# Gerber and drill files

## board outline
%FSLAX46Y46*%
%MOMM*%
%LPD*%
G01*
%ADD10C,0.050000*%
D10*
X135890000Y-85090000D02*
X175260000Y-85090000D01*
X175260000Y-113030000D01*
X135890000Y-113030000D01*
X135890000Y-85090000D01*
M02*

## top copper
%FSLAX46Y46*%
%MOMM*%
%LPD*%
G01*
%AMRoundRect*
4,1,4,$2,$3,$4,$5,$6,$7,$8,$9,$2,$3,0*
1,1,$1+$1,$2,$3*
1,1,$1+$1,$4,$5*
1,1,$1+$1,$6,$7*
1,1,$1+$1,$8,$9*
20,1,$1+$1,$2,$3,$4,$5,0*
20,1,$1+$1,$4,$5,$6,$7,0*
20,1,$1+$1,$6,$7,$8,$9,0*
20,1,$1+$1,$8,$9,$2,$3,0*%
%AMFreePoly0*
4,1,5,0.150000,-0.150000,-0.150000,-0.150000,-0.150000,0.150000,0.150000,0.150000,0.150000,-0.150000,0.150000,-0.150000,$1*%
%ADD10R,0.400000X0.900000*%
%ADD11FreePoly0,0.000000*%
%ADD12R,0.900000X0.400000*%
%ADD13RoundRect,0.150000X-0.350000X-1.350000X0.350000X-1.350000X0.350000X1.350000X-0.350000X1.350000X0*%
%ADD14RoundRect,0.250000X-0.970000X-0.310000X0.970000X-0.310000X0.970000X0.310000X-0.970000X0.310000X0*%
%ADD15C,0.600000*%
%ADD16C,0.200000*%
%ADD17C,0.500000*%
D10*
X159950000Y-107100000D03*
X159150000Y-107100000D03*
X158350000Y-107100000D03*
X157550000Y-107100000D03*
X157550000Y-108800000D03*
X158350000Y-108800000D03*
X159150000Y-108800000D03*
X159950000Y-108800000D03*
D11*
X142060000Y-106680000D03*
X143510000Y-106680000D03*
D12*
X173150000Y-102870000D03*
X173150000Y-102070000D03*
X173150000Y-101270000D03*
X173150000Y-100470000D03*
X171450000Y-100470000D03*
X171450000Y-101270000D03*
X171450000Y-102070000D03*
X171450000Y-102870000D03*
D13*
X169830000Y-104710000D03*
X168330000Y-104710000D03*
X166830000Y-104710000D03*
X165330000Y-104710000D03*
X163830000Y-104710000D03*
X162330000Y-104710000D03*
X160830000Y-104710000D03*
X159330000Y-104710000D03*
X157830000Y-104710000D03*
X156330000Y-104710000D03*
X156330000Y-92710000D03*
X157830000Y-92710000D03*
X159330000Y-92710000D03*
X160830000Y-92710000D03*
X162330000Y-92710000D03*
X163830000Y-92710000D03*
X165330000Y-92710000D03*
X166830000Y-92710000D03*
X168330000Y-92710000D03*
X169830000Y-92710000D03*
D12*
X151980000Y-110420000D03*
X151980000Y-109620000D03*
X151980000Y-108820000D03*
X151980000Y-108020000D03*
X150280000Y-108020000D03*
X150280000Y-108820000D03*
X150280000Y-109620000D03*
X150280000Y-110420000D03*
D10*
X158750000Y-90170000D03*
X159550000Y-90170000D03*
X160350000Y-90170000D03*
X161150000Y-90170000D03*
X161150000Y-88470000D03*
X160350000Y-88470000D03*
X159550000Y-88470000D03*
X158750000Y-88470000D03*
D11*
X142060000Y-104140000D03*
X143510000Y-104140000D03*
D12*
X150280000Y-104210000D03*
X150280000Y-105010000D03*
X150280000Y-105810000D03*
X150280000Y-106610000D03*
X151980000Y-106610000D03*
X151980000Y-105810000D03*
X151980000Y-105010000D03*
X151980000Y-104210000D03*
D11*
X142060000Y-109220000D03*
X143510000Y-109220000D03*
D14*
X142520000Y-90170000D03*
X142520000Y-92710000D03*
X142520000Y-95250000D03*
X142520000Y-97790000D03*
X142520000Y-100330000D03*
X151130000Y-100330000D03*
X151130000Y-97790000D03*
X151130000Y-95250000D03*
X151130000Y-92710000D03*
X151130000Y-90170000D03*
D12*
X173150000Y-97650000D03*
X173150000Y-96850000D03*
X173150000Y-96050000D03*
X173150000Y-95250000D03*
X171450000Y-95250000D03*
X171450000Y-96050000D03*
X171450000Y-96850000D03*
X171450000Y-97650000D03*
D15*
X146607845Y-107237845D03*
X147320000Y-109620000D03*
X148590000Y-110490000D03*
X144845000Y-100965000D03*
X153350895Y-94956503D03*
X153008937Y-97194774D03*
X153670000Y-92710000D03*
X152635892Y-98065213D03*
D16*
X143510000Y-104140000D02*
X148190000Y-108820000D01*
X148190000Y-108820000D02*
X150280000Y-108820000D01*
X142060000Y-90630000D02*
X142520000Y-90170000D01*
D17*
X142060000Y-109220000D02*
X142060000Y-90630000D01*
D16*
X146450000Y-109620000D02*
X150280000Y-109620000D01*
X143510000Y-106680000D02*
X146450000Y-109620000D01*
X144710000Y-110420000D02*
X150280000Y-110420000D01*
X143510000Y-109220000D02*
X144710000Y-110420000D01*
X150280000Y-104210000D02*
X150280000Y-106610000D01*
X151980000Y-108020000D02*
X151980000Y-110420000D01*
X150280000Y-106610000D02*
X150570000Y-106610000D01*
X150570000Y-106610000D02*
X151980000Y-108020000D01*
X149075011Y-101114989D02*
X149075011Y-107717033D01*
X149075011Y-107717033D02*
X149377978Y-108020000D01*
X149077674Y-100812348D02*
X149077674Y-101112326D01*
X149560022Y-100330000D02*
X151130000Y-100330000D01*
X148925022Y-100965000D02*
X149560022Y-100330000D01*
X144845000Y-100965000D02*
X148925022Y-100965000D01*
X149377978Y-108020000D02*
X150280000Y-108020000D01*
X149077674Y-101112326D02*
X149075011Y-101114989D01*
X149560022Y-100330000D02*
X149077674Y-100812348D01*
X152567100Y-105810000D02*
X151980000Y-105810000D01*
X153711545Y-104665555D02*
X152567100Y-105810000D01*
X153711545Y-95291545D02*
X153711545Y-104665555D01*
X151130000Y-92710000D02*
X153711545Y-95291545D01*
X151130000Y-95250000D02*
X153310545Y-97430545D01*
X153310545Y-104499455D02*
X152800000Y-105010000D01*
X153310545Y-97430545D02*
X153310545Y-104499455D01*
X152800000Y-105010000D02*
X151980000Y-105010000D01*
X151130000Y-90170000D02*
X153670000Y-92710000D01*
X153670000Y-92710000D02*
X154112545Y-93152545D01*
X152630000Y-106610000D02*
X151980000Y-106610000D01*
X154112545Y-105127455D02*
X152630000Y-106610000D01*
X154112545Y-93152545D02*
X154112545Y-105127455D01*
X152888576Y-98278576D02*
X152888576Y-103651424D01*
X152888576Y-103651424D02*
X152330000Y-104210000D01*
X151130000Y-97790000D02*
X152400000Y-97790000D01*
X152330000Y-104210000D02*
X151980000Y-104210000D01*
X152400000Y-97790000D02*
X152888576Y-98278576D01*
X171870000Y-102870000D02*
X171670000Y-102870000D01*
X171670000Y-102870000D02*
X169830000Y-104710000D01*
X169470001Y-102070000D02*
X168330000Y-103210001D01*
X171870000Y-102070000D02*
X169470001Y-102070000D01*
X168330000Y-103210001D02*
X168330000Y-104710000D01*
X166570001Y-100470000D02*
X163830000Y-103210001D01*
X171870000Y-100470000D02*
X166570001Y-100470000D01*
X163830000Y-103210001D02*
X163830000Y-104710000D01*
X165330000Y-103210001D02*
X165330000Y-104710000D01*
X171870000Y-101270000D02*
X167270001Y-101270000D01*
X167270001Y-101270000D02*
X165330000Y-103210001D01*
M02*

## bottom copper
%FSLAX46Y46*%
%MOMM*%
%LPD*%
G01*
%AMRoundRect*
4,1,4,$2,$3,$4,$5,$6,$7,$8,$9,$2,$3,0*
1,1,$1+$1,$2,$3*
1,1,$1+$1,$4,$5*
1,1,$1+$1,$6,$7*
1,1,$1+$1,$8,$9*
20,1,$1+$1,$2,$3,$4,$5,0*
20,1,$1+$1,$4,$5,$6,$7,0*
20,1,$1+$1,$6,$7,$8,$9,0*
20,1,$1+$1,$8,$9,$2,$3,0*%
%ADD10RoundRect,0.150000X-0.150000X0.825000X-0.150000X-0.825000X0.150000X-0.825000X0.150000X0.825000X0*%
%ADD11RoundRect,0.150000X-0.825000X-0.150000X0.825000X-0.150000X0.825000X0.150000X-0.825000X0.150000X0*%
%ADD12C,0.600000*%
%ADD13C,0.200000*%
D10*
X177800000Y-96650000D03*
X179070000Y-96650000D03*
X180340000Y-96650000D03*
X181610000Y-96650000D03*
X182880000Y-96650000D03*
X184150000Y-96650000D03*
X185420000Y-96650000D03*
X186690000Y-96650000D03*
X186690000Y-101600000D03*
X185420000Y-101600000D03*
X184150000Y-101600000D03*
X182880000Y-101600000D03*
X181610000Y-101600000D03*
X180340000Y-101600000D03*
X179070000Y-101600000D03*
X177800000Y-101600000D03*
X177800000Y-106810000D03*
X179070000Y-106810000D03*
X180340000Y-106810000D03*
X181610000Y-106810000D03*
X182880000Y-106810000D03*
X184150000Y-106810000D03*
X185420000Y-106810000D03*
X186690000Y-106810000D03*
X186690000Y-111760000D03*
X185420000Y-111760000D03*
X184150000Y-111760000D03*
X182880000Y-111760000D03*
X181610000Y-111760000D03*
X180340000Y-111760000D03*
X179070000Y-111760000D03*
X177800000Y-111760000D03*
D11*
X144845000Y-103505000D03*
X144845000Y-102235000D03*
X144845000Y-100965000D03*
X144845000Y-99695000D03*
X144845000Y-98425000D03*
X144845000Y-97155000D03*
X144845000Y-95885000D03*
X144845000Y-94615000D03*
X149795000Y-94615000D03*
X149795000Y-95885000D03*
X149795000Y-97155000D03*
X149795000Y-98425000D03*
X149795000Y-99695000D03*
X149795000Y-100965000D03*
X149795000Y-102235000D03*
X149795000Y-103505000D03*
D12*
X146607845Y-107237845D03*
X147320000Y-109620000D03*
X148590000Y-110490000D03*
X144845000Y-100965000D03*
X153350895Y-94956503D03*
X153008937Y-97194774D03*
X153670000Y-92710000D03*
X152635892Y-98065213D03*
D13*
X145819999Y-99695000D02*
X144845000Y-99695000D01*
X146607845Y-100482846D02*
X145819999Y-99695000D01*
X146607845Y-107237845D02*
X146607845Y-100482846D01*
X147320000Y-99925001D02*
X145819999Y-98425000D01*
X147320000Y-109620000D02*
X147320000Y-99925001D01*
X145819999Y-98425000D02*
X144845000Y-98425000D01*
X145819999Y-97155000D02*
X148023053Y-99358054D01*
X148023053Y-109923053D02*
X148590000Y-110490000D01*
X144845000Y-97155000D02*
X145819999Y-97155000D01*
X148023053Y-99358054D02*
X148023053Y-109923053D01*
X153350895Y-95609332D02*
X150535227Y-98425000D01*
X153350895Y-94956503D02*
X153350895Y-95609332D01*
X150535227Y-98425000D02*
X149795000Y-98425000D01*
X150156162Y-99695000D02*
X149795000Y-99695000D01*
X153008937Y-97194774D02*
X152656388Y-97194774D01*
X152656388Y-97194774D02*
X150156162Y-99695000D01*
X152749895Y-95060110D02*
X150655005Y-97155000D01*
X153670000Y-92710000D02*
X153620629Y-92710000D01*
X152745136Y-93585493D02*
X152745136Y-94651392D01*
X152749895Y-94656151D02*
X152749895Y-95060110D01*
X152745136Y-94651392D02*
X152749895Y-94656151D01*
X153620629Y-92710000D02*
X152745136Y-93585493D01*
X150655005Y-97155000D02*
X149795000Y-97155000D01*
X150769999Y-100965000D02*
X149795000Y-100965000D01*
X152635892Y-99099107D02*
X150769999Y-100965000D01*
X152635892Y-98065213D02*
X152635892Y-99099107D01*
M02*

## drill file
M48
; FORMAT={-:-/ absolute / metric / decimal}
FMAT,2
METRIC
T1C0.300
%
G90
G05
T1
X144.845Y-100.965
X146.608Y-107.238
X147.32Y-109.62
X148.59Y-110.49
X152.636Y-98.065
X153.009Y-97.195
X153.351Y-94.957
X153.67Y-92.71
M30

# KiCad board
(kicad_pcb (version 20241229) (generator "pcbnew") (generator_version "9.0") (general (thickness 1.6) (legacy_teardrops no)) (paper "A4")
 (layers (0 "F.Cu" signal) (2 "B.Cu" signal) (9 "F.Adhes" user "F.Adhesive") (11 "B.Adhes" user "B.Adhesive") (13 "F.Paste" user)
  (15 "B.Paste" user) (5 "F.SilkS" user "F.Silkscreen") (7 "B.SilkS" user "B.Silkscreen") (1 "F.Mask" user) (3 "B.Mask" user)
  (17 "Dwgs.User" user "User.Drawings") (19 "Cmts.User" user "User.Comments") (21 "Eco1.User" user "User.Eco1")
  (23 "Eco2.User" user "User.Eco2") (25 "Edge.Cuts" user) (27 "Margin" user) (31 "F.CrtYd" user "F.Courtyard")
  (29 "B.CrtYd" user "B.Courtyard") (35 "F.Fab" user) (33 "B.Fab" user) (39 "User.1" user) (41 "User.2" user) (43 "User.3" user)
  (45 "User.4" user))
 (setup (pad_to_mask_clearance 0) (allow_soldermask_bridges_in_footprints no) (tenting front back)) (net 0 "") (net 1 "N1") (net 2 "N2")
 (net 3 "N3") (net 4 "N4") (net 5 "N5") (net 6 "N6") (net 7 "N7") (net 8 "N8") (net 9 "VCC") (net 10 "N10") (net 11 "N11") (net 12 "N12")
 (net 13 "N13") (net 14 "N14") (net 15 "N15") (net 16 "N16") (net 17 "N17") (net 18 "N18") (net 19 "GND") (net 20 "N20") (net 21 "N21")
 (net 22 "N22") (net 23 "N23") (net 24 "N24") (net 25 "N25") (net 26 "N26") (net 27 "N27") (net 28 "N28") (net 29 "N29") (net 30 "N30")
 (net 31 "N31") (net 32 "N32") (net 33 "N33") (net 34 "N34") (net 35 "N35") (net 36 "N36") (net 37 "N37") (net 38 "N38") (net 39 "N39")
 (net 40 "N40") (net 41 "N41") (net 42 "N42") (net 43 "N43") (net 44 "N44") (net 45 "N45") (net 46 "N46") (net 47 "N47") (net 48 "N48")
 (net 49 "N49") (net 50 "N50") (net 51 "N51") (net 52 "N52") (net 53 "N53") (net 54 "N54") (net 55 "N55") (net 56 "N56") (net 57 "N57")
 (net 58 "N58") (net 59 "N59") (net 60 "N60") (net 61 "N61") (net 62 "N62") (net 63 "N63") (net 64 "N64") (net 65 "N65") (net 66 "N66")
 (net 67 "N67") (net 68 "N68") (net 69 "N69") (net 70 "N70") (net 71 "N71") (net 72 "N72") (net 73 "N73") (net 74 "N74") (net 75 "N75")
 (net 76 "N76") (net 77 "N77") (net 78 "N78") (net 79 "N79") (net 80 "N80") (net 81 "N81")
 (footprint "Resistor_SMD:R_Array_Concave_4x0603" (layer "F.Cu") (at 158.75 107.95 -90)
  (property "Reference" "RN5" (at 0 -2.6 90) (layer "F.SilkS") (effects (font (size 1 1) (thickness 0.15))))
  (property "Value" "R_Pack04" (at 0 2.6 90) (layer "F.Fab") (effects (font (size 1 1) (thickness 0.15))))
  (pad "1" smd rect (at -0.85 -1.2 270) (size 0.9 0.4) (layers "F.Cu" "F.Mask" "F.Paste") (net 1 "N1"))
  (pad "2" smd rect (at -0.85 -0.4 270) (size 0.9 0.4) (layers "F.Cu" "F.Mask" "F.Paste") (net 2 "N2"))
  (pad "3" smd rect (at -0.85 0.4 270) (size 0.9 0.4) (layers "F.Cu" "F.Mask" "F.Paste") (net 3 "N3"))
  (pad "4" smd rect (at -0.85 1.2 270) (size 0.9 0.4) (layers "F.Cu" "F.Mask" "F.Paste") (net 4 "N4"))
  (pad "5" smd rect (at 0.85 1.2 270) (size 0.9 0.4) (layers "F.Cu" "F.Mask" "F.Paste") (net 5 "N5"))
  (pad "6" smd rect (at 0.85 0.4 270) (size 0.9 0.4) (layers "F.Cu" "F.Mask" "F.Paste") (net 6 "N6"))
  (pad "7" smd rect (at 0.85 -0.4 270) (size 0.9 0.4) (layers "F.Cu" "F.Mask" "F.Paste") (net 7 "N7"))
  (pad "8" smd rect (at 0.85 -1.2 270) (size 0.9 0.4) (layers "F.Cu" "F.Mask" "F.Paste") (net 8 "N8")))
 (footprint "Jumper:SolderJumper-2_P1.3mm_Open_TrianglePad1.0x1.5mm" (layer "F.Cu") (at 142.785 106.68)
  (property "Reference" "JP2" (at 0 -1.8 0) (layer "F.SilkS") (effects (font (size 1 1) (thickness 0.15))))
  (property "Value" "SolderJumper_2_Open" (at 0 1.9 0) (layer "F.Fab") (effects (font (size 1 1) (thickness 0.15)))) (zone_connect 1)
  (pad "1" smd custom (at -0.725 0) (size 0.3 0.3) (layers "F.Cu" "F.Mask") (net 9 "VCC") (zone_connect 2) (thermal_bridge_angle 45)
   (options (clearance outline) (anchor rect)) (primitives))
  (pad "2" smd custom (at 0.725 0) (size 0.3 0.3) (layers "F.Cu" "F.Mask") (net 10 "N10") (zone_connect 2) (thermal_bridge_angle 45)
   (options (clearance outline) (anchor rect)) (primitives)))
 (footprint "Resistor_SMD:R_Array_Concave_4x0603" (layer "F.Cu") (at 172.3 101.67 180)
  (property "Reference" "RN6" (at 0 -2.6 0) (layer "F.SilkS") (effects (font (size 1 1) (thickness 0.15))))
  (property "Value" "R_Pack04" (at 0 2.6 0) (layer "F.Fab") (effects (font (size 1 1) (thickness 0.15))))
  (pad "1" smd rect (at -0.85 -1.2 180) (size 0.9 0.4) (layers "F.Cu" "F.Mask" "F.Paste") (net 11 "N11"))
  (pad "2" smd rect (at -0.85 -0.4 180) (size 0.9 0.4) (layers "F.Cu" "F.Mask" "F.Paste") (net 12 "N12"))
  (pad "3" smd rect (at -0.85 0.4 180) (size 0.9 0.4) (layers "F.Cu" "F.Mask" "F.Paste") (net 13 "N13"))
  (pad "4" smd rect (at -0.85 1.2 180) (size 0.9 0.4) (layers "F.Cu" "F.Mask" "F.Paste") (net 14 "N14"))
  (pad "5" smd rect (at 0.85 1.2 180) (size 0.9 0.4) (layers "F.Cu" "F.Mask" "F.Paste") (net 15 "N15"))
  (pad "6" smd rect (at 0.85 0.4 180) (size 0.9 0.4) (layers "F.Cu" "F.Mask" "F.Paste") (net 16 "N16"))
  (pad "7" smd rect (at 0.85 -0.4 180) (size 0.9 0.4) (layers "F.Cu" "F.Mask" "F.Paste") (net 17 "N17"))
  (pad "8" smd rect (at 0.85 -1.2 180) (size 0.9 0.4) (layers "F.Cu" "F.Mask" "F.Paste") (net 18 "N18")))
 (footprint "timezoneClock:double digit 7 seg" (layer "F.Cu") (at 163.08 98.71)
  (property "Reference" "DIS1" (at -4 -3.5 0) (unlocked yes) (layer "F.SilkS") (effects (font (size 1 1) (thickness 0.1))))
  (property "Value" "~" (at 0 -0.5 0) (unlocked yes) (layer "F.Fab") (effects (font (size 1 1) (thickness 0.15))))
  (pad "1" smd roundrect (at 6.75 6) (size 1 3) (layers "F.Cu" "F.Mask" "F.Paste") (roundrect_rratio 0.15) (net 18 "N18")
   (thermal_bridge_angle 45))
  (pad "2" smd roundrect (at 5.25 6) (size 1 3) (layers "F.Cu" "F.Mask" "F.Paste") (roundrect_rratio 0.15) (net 17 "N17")
   (thermal_bridge_angle 45))
  (pad "3" smd roundrect (at 3.75 6) (size 1 3) (layers "F.Cu" "F.Mask" "F.Paste") (roundrect_rratio 0.15) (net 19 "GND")
   (thermal_bridge_angle 45))
  (pad "4" smd roundrect (at 2.25 6) (size 1 3) (layers "F.Cu" "F.Mask" "F.Paste") (roundrect_rratio 0.15) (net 16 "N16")
   (thermal_bridge_angle 45))
  (pad "5" smd roundrect (at 0.75 6) (size 1 3) (layers "F.Cu" "F.Mask" "F.Paste") (roundrect_rratio 0.15) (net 15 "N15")
   (thermal_bridge_angle 45))
  (pad "6" smd roundrect (at -0.75 6) (size 1 3) (layers "F.Cu" "F.Mask" "F.Paste") (roundrect_rratio 0.15) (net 8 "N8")
   (thermal_bridge_angle 45))
  (pad "7" smd roundrect (at -2.25 6) (size 1 3) (layers "F.Cu" "F.Mask" "F.Paste") (roundrect_rratio 0.15) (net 7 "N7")
   (thermal_bridge_angle 45))
  (pad "8" smd roundrect (at -3.75 6) (size 1 3) (layers "F.Cu" "F.Mask" "F.Paste") (roundrect_rratio 0.15) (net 19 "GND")
   (thermal_bridge_angle 45))
  (pad "9" smd roundrect (at -5.25 6) (size 1 3) (layers "F.Cu" "F.Mask" "F.Paste") (roundrect_rratio 0.15) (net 6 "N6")
   (thermal_bridge_angle 45))
  (pad "10" smd roundrect (at -6.75 6) (size 1 3) (layers "F.Cu" "F.Mask" "F.Paste") (roundrect_rratio 0.15) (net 5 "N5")
   (thermal_bridge_angle 45))
  (pad "11" smd roundrect (at -6.75 -6) (size 1 3) (layers "F.Cu" "F.Mask" "F.Paste") (roundrect_rratio 0.15) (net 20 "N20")
   (thermal_bridge_angle 45))
  (pad "12" smd roundrect (at -5.25 -6) (size 1 3) (layers "F.Cu" "F.Mask" "F.Paste") (roundrect_rratio 0.15) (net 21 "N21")
   (thermal_bridge_angle 45))
  (pad "13" smd roundrect (at -3.75 -6) (size 1 3) (layers "F.Cu" "F.Mask" "F.Paste") (roundrect_rratio 0.15) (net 19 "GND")
   (thermal_bridge_angle 45))
  (pad "14" smd roundrect (at -2.25 -6) (size 1 3) (layers "F.Cu" "F.Mask" "F.Paste") (roundrect_rratio 0.15) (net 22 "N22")
   (thermal_bridge_angle 45))
  (pad "15" smd roundrect (at -0.75 -6) (size 1 3) (layers "F.Cu" "F.Mask" "F.Paste") (roundrect_rratio 0.15) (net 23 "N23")
   (thermal_bridge_angle 45))
  (pad "16" smd roundrect (at 0.75 -6) (size 1 3) (layers "F.Cu" "F.Mask" "F.Paste") (roundrect_rratio 0.15) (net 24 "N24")
   (thermal_bridge_angle 45))
  (pad "17" smd roundrect (at 2.25 -6) (size 1 3) (layers "F.Cu" "F.Mask" "F.Paste") (roundrect_rratio 0.15) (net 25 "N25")
   (thermal_bridge_angle 45))
  (pad "18" smd roundrect (at 3.75 -6) (size 1 3) (layers "F.Cu" "F.Mask" "F.Paste") (roundrect_rratio 0.15) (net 19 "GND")
   (thermal_bridge_angle 45))
  (pad "19" smd roundrect (at 5.25 -6) (size 1 3) (layers "F.Cu" "F.Mask" "F.Paste") (roundrect_rratio 0.15) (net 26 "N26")
   (thermal_bridge_angle 45))
  (pad "20" smd roundrect (at 6.75 -6) (size 1 3) (layers "F.Cu" "F.Mask" "F.Paste") (roundrect_rratio 0.15) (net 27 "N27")
   (thermal_bridge_angle 45)))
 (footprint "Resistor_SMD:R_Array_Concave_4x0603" (layer "F.Cu") (at 151.13 109.22 180)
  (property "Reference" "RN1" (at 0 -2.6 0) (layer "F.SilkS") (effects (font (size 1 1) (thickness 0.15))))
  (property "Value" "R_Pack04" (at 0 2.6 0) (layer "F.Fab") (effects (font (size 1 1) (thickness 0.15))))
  (pad "1" smd rect (at -0.85 -1.2 180) (size 0.9 0.4) (layers "F.Cu" "F.Mask" "F.Paste") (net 19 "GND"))
  (pad "2" smd rect (at -0.85 -0.4 180) (size 0.9 0.4) (layers "F.Cu" "F.Mask" "F.Paste") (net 19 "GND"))
  (pad "3" smd rect (at -0.85 0.4 180) (size 0.9 0.4) (layers "F.Cu" "F.Mask" "F.Paste") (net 19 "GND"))
  (pad "4" smd rect (at -0.85 1.2 180) (size 0.9 0.4) (layers "F.Cu" "F.Mask" "F.Paste") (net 19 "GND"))
  (pad "5" smd rect (at 0.85 1.2 180) (size 0.9 0.4) (layers "F.Cu" "F.Mask" "F.Paste") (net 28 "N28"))
  (pad "6" smd rect (at 0.85 0.4 180) (size 0.9 0.4) (layers "F.Cu" "F.Mask" "F.Paste") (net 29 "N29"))
  (pad "7" smd rect (at 0.85 -0.4 180) (size 0.9 0.4) (layers "F.Cu" "F.Mask" "F.Paste") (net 10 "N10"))
  (pad "8" smd rect (at 0.85 -1.2 180) (size 0.9 0.4) (layers "F.Cu" "F.Mask" "F.Paste") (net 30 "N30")))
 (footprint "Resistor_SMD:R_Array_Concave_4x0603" (layer "F.Cu") (at 159.95 89.32 90)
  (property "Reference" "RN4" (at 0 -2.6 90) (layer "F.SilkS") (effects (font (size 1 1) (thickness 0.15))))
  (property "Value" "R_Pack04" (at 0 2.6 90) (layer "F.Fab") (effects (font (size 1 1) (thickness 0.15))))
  (pad "1" smd rect (at -0.85 -1.2 90) (size 0.9 0.4) (layers "F.Cu" "F.Mask" "F.Paste") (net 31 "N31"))
  (pad "2" smd rect (at -0.85 -0.4 90) (size 0.9 0.4) (layers "F.Cu" "F.Mask" "F.Paste") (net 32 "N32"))
  (pad "3" smd rect (at -0.85 0.4 90) (size 0.9 0.4) (layers "F.Cu" "F.Mask" "F.Paste") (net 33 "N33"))
  (pad "4" smd rect (at -0.85 1.2 90) (size 0.9 0.4) (layers "F.Cu" "F.Mask" "F.Paste") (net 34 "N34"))
  (pad "5" smd rect (at 0.85 1.2 90) (size 0.9 0.4) (layers "F.Cu" "F.Mask" "F.Paste") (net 23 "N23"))
  (pad "6" smd rect (at 0.85 0.4 90) (size 0.9 0.4) (layers "F.Cu" "F.Mask" "F.Paste") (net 22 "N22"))
  (pad "7" smd rect (at 0.85 -0.4 90) (size 0.9 0.4) (layers "F.Cu" "F.Mask" "F.Paste") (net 21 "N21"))
  (pad "8" smd rect (at 0.85 -1.2 90) (size 0.9 0.4) (layers "F.Cu" "F.Mask" "F.Paste") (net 20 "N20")))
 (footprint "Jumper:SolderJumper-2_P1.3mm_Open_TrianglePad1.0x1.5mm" (layer "F.Cu") (at 142.785 104.14)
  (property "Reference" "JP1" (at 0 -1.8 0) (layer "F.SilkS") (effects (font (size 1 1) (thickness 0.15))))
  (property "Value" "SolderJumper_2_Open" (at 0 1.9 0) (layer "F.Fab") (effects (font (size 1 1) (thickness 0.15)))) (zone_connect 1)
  (pad "1" smd custom (at -0.725 0) (size 0.3 0.3) (layers "F.Cu" "F.Mask") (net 9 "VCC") (zone_connect 2) (thermal_bridge_angle 45)
   (options (clearance outline) (anchor rect)) (primitives))
  (pad "2" smd custom (at 0.725 0) (size 0.3 0.3) (layers "F.Cu" "F.Mask") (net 29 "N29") (zone_connect 2) (thermal_bridge_angle 45)
   (options (clearance outline) (anchor rect)) (primitives)))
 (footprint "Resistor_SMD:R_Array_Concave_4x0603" (layer "F.Cu") (at 151.13 105.41)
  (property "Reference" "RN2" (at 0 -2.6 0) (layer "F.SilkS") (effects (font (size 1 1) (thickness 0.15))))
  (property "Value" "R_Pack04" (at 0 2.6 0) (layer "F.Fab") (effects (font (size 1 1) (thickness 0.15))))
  (pad "1" smd rect (at -0.85 -1.2) (size 0.9 0.4) (layers "F.Cu" "F.Mask" "F.Paste") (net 19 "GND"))
  (pad "2" smd rect (at -0.85 -0.4) (size 0.9 0.4) (layers "F.Cu" "F.Mask" "F.Paste") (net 19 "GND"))
  (pad "3" smd rect (at -0.85 0.4) (size 0.9 0.4) (layers "F.Cu" "F.Mask" "F.Paste") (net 19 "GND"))
  (pad "4" smd rect (at -0.85 1.2) (size 0.9 0.4) (layers "F.Cu" "F.Mask" "F.Paste") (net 19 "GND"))
  (pad "5" smd rect (at 0.85 1.2) (size 0.9 0.4) (layers "F.Cu" "F.Mask" "F.Paste") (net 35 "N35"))
  (pad "6" smd rect (at 0.85 0.4) (size 0.9 0.4) (layers "F.Cu" "F.Mask" "F.Paste") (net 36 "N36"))
  (pad "7" smd rect (at 0.85 -0.4) (size 0.9 0.4) (layers "F.Cu" "F.Mask" "F.Paste") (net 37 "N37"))
  (pad "8" smd rect (at 0.85 -1.2) (size 0.9 0.4) (layers "F.Cu" "F.Mask" "F.Paste") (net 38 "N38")))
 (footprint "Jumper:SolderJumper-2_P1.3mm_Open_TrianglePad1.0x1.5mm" (layer "F.Cu") (at 142.785 109.22)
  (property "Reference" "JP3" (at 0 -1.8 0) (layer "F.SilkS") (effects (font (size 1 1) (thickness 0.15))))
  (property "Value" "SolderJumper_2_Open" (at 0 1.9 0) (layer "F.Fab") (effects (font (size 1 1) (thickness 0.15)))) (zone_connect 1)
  (pad "1" smd custom (at -0.725 0) (size 0.3 0.3) (layers "F.Cu" "F.Mask") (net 9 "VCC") (zone_connect 2) (thermal_bridge_angle 45)
   (options (clearance outline) (anchor rect)) (primitives))
  (pad "2" smd custom (at 0.725 0) (size 0.3 0.3) (layers "F.Cu" "F.Mask") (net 30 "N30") (zone_connect 2) (thermal_bridge_angle 45)
   (options (clearance outline) (anchor rect)) (primitives)))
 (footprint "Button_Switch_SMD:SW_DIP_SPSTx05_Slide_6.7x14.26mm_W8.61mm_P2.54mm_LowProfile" (layer "F.Cu") (at 146.825 95.25)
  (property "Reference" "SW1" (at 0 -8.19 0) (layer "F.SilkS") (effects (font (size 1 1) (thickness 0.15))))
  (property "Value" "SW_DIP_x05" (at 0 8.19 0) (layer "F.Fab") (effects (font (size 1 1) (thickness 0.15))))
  (pad "1" smd roundrect (at -4.305 -5.08) (size 2.44 1.12) (layers "F.Cu" "F.Mask" "F.Paste") (roundrect_rratio 0.223214) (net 9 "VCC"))
  (pad "2" smd roundrect (at -4.305 -2.54) (size 2.44 1.12) (layers "F.Cu" "F.Mask" "F.Paste") (roundrect_rratio 0.223214) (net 9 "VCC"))
  (pad "3" smd roundrect (at -4.305 0) (size 2.44 1.12) (layers "F.Cu" "F.Mask" "F.Paste") (roundrect_rratio 0.223214) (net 9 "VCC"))
  (pad "4" smd roundrect (at -4.305 2.54) (size 2.44 1.12) (layers "F.Cu" "F.Mask" "F.Paste") (roundrect_rratio 0.223214) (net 9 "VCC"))
  (pad "5" smd roundrect (at -4.305 5.08) (size 2.44 1.12) (layers "F.Cu" "F.Mask" "F.Paste") (roundrect_rratio 0.223214) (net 9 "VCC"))
  (pad "6" smd roundrect (at 4.305 5.08) (size 2.44 1.12) (layers "F.Cu" "F.Mask" "F.Paste") (roundrect_rratio 0.223214) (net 28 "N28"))
  (pad "7" smd roundrect (at 4.305 2.54) (size 2.44 1.12) (layers "F.Cu" "F.Mask" "F.Paste") (roundrect_rratio 0.223214) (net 38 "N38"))
  (pad "8" smd roundrect (at 4.305 0) (size 2.44 1.12) (layers "F.Cu" "F.Mask" "F.Paste") (roundrect_rratio 0.223214) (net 37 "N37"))
  (pad "9" smd roundrect (at 4.305 -2.54) (size 2.44 1.12) (layers "F.Cu" "F.Mask" "F.Paste") (roundrect_rratio 0.223214) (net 36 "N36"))
  (pad "10" smd roundrect (at 4.305 -5.08) (size 2.44 1.12) (layers "F.Cu" "F.Mask" "F.Paste") (roundrect_rratio 0.223214) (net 35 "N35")))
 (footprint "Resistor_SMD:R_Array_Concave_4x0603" (layer "F.Cu") (at 172.3 96.45 180)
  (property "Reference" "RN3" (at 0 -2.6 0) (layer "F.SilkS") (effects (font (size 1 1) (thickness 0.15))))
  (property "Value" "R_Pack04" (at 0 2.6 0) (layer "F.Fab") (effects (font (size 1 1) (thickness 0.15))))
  (pad "1" smd rect (at -0.85 -1.2 180) (size 0.9 0.4) (layers "F.Cu" "F.Mask" "F.Paste") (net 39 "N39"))
  (pad "2" smd rect (at -0.85 -0.4 180) (size 0.9 0.4) (layers "F.Cu" "F.Mask" "F.Paste") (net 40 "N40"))
  (pad "3" smd rect (at -0.85 0.4 180) (size 0.9 0.4) (layers "F.Cu" "F.Mask" "F.Paste") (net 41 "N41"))
  (pad "4" smd rect (at -0.85 1.2 180) (size 0.9 0.4) (layers "F.Cu" "F.Mask" "F.Paste") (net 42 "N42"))
  (pad "5" smd rect (at 0.85 1.2 180) (size 0.9 0.4) (layers "F.Cu" "F.Mask" "F.Paste") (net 27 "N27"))
  (pad "6" smd rect (at 0.85 0.4 180) (size 0.9 0.4) (layers "F.Cu" "F.Mask" "F.Paste") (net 26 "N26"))
  (pad "7" smd rect (at 0.85 -0.4 180) (size 0.9 0.4) (layers "F.Cu" "F.Mask" "F.Paste") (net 25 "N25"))
  (pad "8" smd rect (at 0.85 -1.2 180) (size 0.9 0.4) (layers "F.Cu" "F.Mask" "F.Paste") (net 24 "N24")))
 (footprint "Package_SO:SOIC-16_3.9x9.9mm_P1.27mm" (layer "B.Cu") (at 182.245 99.125 -90)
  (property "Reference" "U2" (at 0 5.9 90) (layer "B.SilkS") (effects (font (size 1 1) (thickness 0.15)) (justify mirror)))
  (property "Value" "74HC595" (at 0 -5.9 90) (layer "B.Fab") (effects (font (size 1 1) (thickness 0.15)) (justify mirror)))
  (pad "1" smd roundrect (at -2.475 4.445 270) (size 1.95 0.6) (layers "B.Cu" "B.Mask" "B.Paste") (roundrect_rratio 0.25) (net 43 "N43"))
  (pad "2" smd roundrect (at -2.475 3.175 270) (size 1.95 0.6) (layers "B.Cu" "B.Mask" "B.Paste") (roundrect_rratio 0.25) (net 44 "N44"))
  (pad "3" smd roundrect (at -2.475 1.905 270) (size 1.95 0.6) (layers "B.Cu" "B.Mask" "B.Paste") (roundrect_rratio 0.25) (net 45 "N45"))
  (pad "4" smd roundrect (at -2.475 0.635 270) (size 1.95 0.6) (layers "B.Cu" "B.Mask" "B.Paste") (roundrect_rratio 0.25) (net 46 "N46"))
  (pad "5" smd roundrect (at -2.475 -0.635 270) (size 1.95 0.6) (layers "B.Cu" "B.Mask" "B.Paste") (roundrect_rratio 0.25) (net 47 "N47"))
  (pad "6" smd roundrect (at -2.475 -1.905 270) (size 1.95 0.6) (layers "B.Cu" "B.Mask" "B.Paste") (roundrect_rratio 0.25) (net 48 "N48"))
  (pad "7" smd roundrect (at -2.475 -3.175 270) (size 1.95 0.6) (layers "B.Cu" "B.Mask" "B.Paste") (roundrect_rratio 0.25) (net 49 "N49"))
  (pad "8" smd roundrect (at -2.475 -4.445 270) (size 1.95 0.6) (layers "B.Cu" "B.Mask" "B.Paste") (roundrect_rratio 0.25) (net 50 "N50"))
  (pad "9" smd roundrect (at 2.475 -4.445 270) (size 1.95 0.6) (layers "B.Cu" "B.Mask" "B.Paste") (roundrect_rratio 0.25) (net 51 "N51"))
  (pad "10" smd roundrect (at 2.475 -3.175 270) (size 1.95 0.6) (layers "B.Cu" "B.Mask" "B.Paste") (roundrect_rratio 0.25) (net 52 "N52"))
  (pad "11" smd roundrect (at 2.475 -1.905 270) (size 1.95 0.6) (layers "B.Cu" "B.Mask" "B.Paste") (roundrect_rratio 0.25) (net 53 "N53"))
  (pad "12" smd roundrect (at 2.475 -0.635 270) (size 1.95 0.6) (layers "B.Cu" "B.Mask" "B.Paste") (roundrect_rratio 0.25) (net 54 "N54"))
  (pad "13" smd roundrect (at 2.475 0.635 270) (size 1.95 0.6) (layers "B.Cu" "B.Mask" "B.Paste") (roundrect_rratio 0.25) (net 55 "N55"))
  (pad "14" smd roundrect (at 2.475 1.905 270) (size 1.95 0.6) (layers "B.Cu" "B.Mask" "B.Paste") (roundrect_rratio 0.25) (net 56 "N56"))
  (pad "15" smd roundrect (at 2.475 3.175 270) (size 1.95 0.6) (layers "B.Cu" "B.Mask" "B.Paste") (roundrect_rratio 0.25) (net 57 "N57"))
  (pad "16" smd roundrect (at 2.475 4.445 270) (size 1.95 0.6) (layers "B.Cu" "B.Mask" "B.Paste") (roundrect_rratio 0.25) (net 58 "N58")))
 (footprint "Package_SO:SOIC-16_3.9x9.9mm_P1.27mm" (layer "B.Cu") (at 182.245 109.285 -90)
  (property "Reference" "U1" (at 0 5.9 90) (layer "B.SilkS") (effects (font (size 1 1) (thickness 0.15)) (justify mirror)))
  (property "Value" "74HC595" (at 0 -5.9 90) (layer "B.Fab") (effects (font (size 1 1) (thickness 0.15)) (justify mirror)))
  (pad "1" smd roundrect (at -2.475 4.445 270) (size 1.95 0.6) (layers "B.Cu" "B.Mask" "B.Paste") (roundrect_rratio 0.25) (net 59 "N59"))
  (pad "2" smd roundrect (at -2.475 3.175 270) (size 1.95 0.6) (layers "B.Cu" "B.Mask" "B.Paste") (roundrect_rratio 0.25) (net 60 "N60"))
  (pad "3" smd roundrect (at -2.475 1.905 270) (size 1.95 0.6) (layers "B.Cu" "B.Mask" "B.Paste") (roundrect_rratio 0.25) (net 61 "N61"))
  (pad "4" smd roundrect (at -2.475 0.635 270) (size 1.95 0.6) (layers "B.Cu" "B.Mask" "B.Paste") (roundrect_rratio 0.25) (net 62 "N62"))
  (pad "5" smd roundrect (at -2.475 -0.635 270) (size 1.95 0.6) (layers "B.Cu" "B.Mask" "B.Paste") (roundrect_rratio 0.25) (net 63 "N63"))
  (pad "6" smd roundrect (at -2.475 -1.905 270) (size 1.95 0.6) (layers "B.Cu" "B.Mask" "B.Paste") (roundrect_rratio 0.25) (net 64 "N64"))
  (pad "7" smd roundrect (at -2.475 -3.175 270) (size 1.95 0.6) (layers "B.Cu" "B.Mask" "B.Paste") (roundrect_rratio 0.25) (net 56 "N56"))
  (pad "8" smd roundrect (at -2.475 -4.445 270) (size 1.95 0.6) (layers "B.Cu" "B.Mask" "B.Paste") (roundrect_rratio 0.25) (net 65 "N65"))
  (pad "9" smd roundrect (at 2.475 -4.445 270) (size 1.95 0.6) (layers "B.Cu" "B.Mask" "B.Paste") (roundrect_rratio 0.25) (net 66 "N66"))
  (pad "10" smd roundrect (at 2.475 -3.175 270) (size 1.95 0.6) (layers "B.Cu" "B.Mask" "B.Paste") (roundrect_rratio 0.25) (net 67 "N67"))
  (pad "11" smd roundrect (at 2.475 -1.905 270) (size 1.95 0.6) (layers "B.Cu" "B.Mask" "B.Paste") (roundrect_rratio 0.25) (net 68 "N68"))
  (pad "12" smd roundrect (at 2.475 -0.635 270) (size 1.95 0.6) (layers "B.Cu" "B.Mask" "B.Paste") (roundrect_rratio 0.25) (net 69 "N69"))
  (pad "13" smd roundrect (at 2.475 0.635 270) (size 1.95 0.6) (layers "B.Cu" "B.Mask" "B.Paste") (roundrect_rratio 0.25) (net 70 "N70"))
  (pad "14" smd roundrect (at 2.475 1.905 270) (size 1.95 0.6) (layers "B.Cu" "B.Mask" "B.Paste") (roundrect_rratio 0.25) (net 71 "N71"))
  (pad "15" smd roundrect (at 2.475 3.175 270) (size 1.95 0.6) (layers "B.Cu" "B.Mask" "B.Paste") (roundrect_rratio 0.25) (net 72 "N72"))
  (pad "16" smd roundrect (at 2.475 4.445 270) (size 1.95 0.6) (layers "B.Cu" "B.Mask" "B.Paste") (roundrect_rratio 0.25) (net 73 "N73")))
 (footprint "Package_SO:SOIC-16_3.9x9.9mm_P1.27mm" (layer "B.Cu") (at 147.32 99.06)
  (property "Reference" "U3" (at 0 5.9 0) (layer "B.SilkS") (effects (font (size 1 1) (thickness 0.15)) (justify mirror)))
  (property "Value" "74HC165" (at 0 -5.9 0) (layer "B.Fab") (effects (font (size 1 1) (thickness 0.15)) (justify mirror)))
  (pad "1" smd roundrect (at -2.475 4.445) (size 1.95 0.6) (layers "B.Cu" "B.Mask" "B.Paste") (roundrect_rratio 0.25) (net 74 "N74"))
  (pad "2" smd roundrect (at -2.475 3.175) (size 1.95 0.6) (layers "B.Cu" "B.Mask" "B.Paste") (roundrect_rratio 0.25) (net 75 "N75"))
  (pad "3" smd roundrect (at -2.475 1.905) (size 1.95 0.6) (layers "B.Cu" "B.Mask" "B.Paste") (roundrect_rratio 0.25) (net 28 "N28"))
  (pad "4" smd roundrect (at -2.475 0.635) (size 1.95 0.6) (layers "B.Cu" "B.Mask" "B.Paste") (roundrect_rratio 0.25) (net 29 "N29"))
  (pad "5" smd roundrect (at -2.475 -0.635) (size 1.95 0.6) (layers "B.Cu" "B.Mask" "B.Paste") (roundrect_rratio 0.25) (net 10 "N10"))
  (pad "6" smd roundrect (at -2.475 -1.905) (size 1.95 0.6) (layers "B.Cu" "B.Mask" "B.Paste") (roundrect_rratio 0.25) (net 30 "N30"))
  (pad "7" smd roundrect (at -2.475 -3.175) (size 1.95 0.6) (layers "B.Cu" "B.Mask" "B.Paste") (roundrect_rratio 0.25) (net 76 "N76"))
  (pad "8" smd roundrect (at -2.475 -4.445) (size 1.95 0.6) (layers "B.Cu" "B.Mask" "B.Paste") (roundrect_rratio 0.25) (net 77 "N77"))
  (pad "9" smd roundrect (at 2.475 -4.445) (size 1.95 0.6) (layers "B.Cu" "B.Mask" "B.Paste") (roundrect_rratio 0.25) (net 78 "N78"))
  (pad "10" smd roundrect (at 2.475 -3.175) (size 1.95 0.6) (layers "B.Cu" "B.Mask" "B.Paste") (roundrect_rratio 0.25) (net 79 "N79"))
  (pad "11" smd roundrect (at 2.475 -1.905) (size 1.95 0.6) (layers "B.Cu" "B.Mask" "B.Paste") (roundrect_rratio 0.25) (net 35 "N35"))
  (pad "12" smd roundrect (at 2.475 -0.635) (size 1.95 0.6) (layers "B.Cu" "B.Mask" "B.Paste") (roundrect_rratio 0.25) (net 36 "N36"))
  (pad "13" smd roundrect (at 2.475 0.635) (size 1.95 0.6) (layers "B.Cu" "B.Mask" "B.Paste") (roundrect_rratio 0.25) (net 37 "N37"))
  (pad "14" smd roundrect (at 2.475 1.905) (size 1.95 0.6) (layers "B.Cu" "B.Mask" "B.Paste") (roundrect_rratio 0.25) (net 38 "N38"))
  (pad "15" smd roundrect (at 2.475 3.175) (size 1.95 0.6) (layers "B.Cu" "B.Mask" "B.Paste") (roundrect_rratio 0.25) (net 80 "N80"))
  (pad "16" smd roundrect (at 2.475 4.445) (size 1.95 0.6) (layers "B.Cu" "B.Mask" "B.Paste") (roundrect_rratio 0.25) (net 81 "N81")))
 (gr_rect (start 135.89 85.09) (end 175.26 113.03) (stroke (width 0.05) (type default)) (fill no) (layer "Edge.Cuts"))
 (segment (start 143.51 104.14) (end 148.19 108.82) (width 0.2) (layer "F.Cu") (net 29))
 (segment (start 148.19 108.82) (end 150.28 108.82) (width 0.2) (layer "F.Cu") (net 29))
 (via (at 146.607845 107.237845) (size 0.6) (drill 0.3) (layers "F.Cu" "B.Cu") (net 29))
 (segment (start 145.819999 99.695) (end 144.845 99.695) (width 0.2) (layer "B.Cu") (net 29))
 (segment (start 146.607845 100.482846) (end 145.819999 99.695) (width 0.2) (layer "B.Cu") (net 29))
 (segment (start 146.607845 107.237845) (end 146.607845 100.482846) (width 0.2) (layer "B.Cu") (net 29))
 (segment (start 142.06 90.63) (end 142.52 90.17) (width 0.2) (layer "F.Cu") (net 9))
 (segment (start 142.06 109.22) (end 142.06 90.63) (width 0.5) (layer "F.Cu") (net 9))
 (segment (start 146.45 109.62) (end 150.28 109.62) (width 0.2) (layer "F.Cu") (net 10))
 (segment (start 143.51 106.68) (end 146.45 109.62) (width 0.2) (layer "F.Cu") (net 10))
 (via (at 147.32 109.62) (size 0.6) (drill 0.3) (layers "F.Cu" "B.Cu") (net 10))
 (segment (start 147.32 99.925001) (end 145.819999 98.425) (width 0.2) (layer "B.Cu") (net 10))
 (segment (start 147.32 109.62) (end 147.32 99.925001) (width 0.2) (layer "B.Cu") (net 10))
 (segment (start 145.819999 98.425) (end 144.845 98.425) (width 0.2) (layer "B.Cu") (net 10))
 (segment (start 144.71 110.42) (end 150.28 110.42) (width 0.2) (layer "F.Cu") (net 30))
 (segment (start 143.51 109.22) (end 144.71 110.42) (width 0.2) (layer "F.Cu") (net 30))
 (via (at 148.59 110.49) (size 0.6) (drill 0.3) (layers "F.Cu" "B.Cu") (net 30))
 (segment (start 145.819999 97.155) (end 148.023053 99.358054) (width 0.2) (layer "B.Cu") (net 30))
 (segment (start 148.023053 109.923053) (end 148.59 110.49) (width 0.2) (layer "B.Cu") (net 30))
 (segment (start 144.845 97.155) (end 145.819999 97.155) (width 0.2) (layer "B.Cu") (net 30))
 (segment (start 148.023053 99.358054) (end 148.023053 109.923053) (width 0.2) (layer "B.Cu") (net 30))
 (segment (start 150.28 104.21) (end 150.28 106.61) (width 0.2) (layer "F.Cu") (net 19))
 (segment (start 151.98 108.02) (end 151.98 110.42) (width 0.2) (layer "F.Cu") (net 19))
 (segment (start 150.28 106.61) (end 150.57 106.61) (width 0.2) (layer "F.Cu") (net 19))
 (segment (start 150.57 106.61) (end 151.98 108.02) (width 0.2) (layer "F.Cu") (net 19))
 (segment (start 149.075011 101.114989) (end 149.075011 107.717033) (width 0.2) (layer "F.Cu") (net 28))
 (segment (start 149.075011 107.717033) (end 149.377978 108.02) (width 0.2) (layer "F.Cu") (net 28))
 (segment (start 149.077674 100.812348) (end 149.077674 101.112326) (width 0.2) (layer "F.Cu") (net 28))
 (segment (start 149.560022 100.33) (end 151.13 100.33) (width 0.2) (layer "F.Cu") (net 28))
 (segment (start 148.925022 100.965) (end 149.560022 100.33) (width 0.2) (layer "F.Cu") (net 28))
 (segment (start 144.845 100.965) (end 148.925022 100.965) (width 0.2) (layer "F.Cu") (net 28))
 (segment (start 149.377978 108.02) (end 150.28 108.02) (width 0.2) (layer "F.Cu") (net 28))
 (segment (start 149.077674 101.112326) (end 149.075011 101.114989) (width 0.2) (layer "F.Cu") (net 28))
 (segment (start 149.560022 100.33) (end 149.077674 100.812348) (width 0.2) (layer "F.Cu") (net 28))
 (via (at 144.845 100.965) (size 0.6) (drill 0.3) (layers "F.Cu" "B.Cu") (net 28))
 (segment (start 152.5671 105.81) (end 151.98 105.81) (width 0.2) (layer "F.Cu") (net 36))
 (segment (start 153.711545 104.665555) (end 152.5671 105.81) (width 0.2) (layer "F.Cu") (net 36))
 (segment (start 153.711545 95.291545) (end 153.711545 104.665555) (width 0.2) (layer "F.Cu") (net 36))
 (segment (start 151.13 92.71) (end 153.711545 95.291545) (width 0.2) (layer "F.Cu") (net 36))
 (via (at 153.350895 94.956503) (size 0.6) (drill 0.3) (layers "F.Cu" "B.Cu") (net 36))
 (segment (start 153.350895 95.609332) (end 150.535227 98.425) (width 0.2) (layer "B.Cu") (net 36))
 (segment (start 153.350895 94.956503) (end 153.350895 95.609332) (width 0.2) (layer "B.Cu") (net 36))
 (segment (start 150.535227 98.425) (end 149.795 98.425) (width 0.2) (layer "B.Cu") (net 36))
 (segment (start 151.13 95.25) (end 153.310545 97.430545) (width 0.2) (layer "F.Cu") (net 37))
 (segment (start 153.310545 104.499455) (end 152.8 105.01) (width 0.2) (layer "F.Cu") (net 37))
 (segment (start 153.310545 97.430545) (end 153.310545 104.499455) (width 0.2) (layer "F.Cu") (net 37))
 (segment (start 152.8 105.01) (end 151.98 105.01) (width 0.2) (layer "F.Cu") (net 37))
 (via (at 153.008937 97.194774) (size 0.6) (drill 0.3) (layers "F.Cu" "B.Cu") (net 37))
 (segment (start 150.156162 99.695) (end 149.795 99.695) (width 0.2) (layer "B.Cu") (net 37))
 (segment (start 153.008937 97.194774) (end 152.656388 97.194774) (width 0.2) (layer "B.Cu") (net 37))
 (segment (start 152.656388 97.194774) (end 150.156162 99.695) (width 0.2) (layer "B.Cu") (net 37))
 (segment (start 151.13 90.17) (end 153.67 92.71) (width 0.2) (layer "F.Cu") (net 35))
 (segment (start 153.67 92.71) (end 154.112545 93.152545) (width 0.2) (layer "F.Cu") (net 35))
 (segment (start 152.63 106.61) (end 151.98 106.61) (width 0.2) (layer "F.Cu") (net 35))
 (segment (start 154.112545 105.127455) (end 152.63 106.61) (width 0.2) (layer "F.Cu") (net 35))
 (segment (start 154.112545 93.152545) (end 154.112545 105.127455) (width 0.2) (layer "F.Cu") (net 35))
 (via (at 153.67 92.71) (size 0.6) (drill 0.3) (layers "F.Cu" "B.Cu") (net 35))
 (segment (start 152.749895 95.06011) (end 150.655005 97.155) (width 0.2) (layer "B.Cu") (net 35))
 (segment (start 153.67 92.71) (end 153.620629 92.71) (width 0.2) (layer "B.Cu") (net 35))
 (segment (start 152.745136 93.585493) (end 152.745136 94.651392) (width 0.2) (layer "B.Cu") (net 35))
 (segment (start 152.749895 94.656151) (end 152.749895 95.06011) (width 0.2) (layer "B.Cu") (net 35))
 (segment (start 152.745136 94.651392) (end 152.749895 94.656151) (width 0.2) (layer "B.Cu") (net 35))
 (segment (start 153.620629 92.71) (end 152.745136 93.585493) (width 0.2) (layer "B.Cu") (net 35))
 (segment (start 150.655005 97.155) (end 149.795 97.155) (width 0.2) (layer "B.Cu") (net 35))
 (segment (start 152.888576 98.278576) (end 152.888576 103.651424) (width 0.2) (layer "F.Cu") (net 38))
 (segment (start 152.888576 103.651424) (end 152.33 104.21) (width 0.2) (layer "F.Cu") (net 38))
 (segment (start 151.13 97.79) (end 152.4 97.79) (width 0.2) (layer "F.Cu") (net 38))
 (segment (start 152.33 104.21) (end 151.98 104.21) (width 0.2) (layer "F.Cu") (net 38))
 (segment (start 152.4 97.79) (end 152.888576 98.278576) (width 0.2) (layer "F.Cu") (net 38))
 (via (at 152.635892 98.065213) (size 0.6) (drill 0.3) (layers "F.Cu" "B.Cu") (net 38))
 (segment (start 150.769999 100.965) (end 149.795 100.965) (width 0.2) (layer "B.Cu") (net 38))
 (segment (start 152.635892 99.099107) (end 150.769999 100.965) (width 0.2) (layer "B.Cu") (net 38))
 (segment (start 152.635892 98.065213) (end 152.635892 99.099107) (width 0.2) (layer "B.Cu") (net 38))
 (segment (start 171.87 102.87) (end 171.67 102.87) (width 0.2) (layer "F.Cu") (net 18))
 (segment (start 171.67 102.87) (end 169.83 104.71) (width 0.2) (layer "F.Cu") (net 18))
 (segment (start 169.470001 102.07) (end 168.33 103.210001) (width 0.2) (layer "F.Cu") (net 17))
 (segment (start 171.87 102.07) (end 169.470001 102.07) (width 0.2) (layer "F.Cu") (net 17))
 (segment (start 168.33 103.210001) (end 168.33 104.71) (width 0.2) (layer "F.Cu") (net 17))
 (segment (start 166.570001 100.47) (end 163.83 103.210001) (width 0.2) (layer "F.Cu") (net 15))
 (segment (start 171.87 100.47) (end 166.570001 100.47) (width 0.2) (layer "F.Cu") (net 15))
 (segment (start 163.83 103.210001) (end 163.83 104.71) (width 0.2) (layer "F.Cu") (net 15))
 (segment (start 165.33 103.210001) (end 165.33 104.71) (width 0.2) (layer "F.Cu") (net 16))
 (segment (start 171.87 101.27) (end 167.270001 101.27) (width 0.2) (layer "F.Cu") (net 16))
 (segment (start 167.270001 101.27) (end 165.33 103.210001) (width 0.2) (layer "F.Cu") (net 16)))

